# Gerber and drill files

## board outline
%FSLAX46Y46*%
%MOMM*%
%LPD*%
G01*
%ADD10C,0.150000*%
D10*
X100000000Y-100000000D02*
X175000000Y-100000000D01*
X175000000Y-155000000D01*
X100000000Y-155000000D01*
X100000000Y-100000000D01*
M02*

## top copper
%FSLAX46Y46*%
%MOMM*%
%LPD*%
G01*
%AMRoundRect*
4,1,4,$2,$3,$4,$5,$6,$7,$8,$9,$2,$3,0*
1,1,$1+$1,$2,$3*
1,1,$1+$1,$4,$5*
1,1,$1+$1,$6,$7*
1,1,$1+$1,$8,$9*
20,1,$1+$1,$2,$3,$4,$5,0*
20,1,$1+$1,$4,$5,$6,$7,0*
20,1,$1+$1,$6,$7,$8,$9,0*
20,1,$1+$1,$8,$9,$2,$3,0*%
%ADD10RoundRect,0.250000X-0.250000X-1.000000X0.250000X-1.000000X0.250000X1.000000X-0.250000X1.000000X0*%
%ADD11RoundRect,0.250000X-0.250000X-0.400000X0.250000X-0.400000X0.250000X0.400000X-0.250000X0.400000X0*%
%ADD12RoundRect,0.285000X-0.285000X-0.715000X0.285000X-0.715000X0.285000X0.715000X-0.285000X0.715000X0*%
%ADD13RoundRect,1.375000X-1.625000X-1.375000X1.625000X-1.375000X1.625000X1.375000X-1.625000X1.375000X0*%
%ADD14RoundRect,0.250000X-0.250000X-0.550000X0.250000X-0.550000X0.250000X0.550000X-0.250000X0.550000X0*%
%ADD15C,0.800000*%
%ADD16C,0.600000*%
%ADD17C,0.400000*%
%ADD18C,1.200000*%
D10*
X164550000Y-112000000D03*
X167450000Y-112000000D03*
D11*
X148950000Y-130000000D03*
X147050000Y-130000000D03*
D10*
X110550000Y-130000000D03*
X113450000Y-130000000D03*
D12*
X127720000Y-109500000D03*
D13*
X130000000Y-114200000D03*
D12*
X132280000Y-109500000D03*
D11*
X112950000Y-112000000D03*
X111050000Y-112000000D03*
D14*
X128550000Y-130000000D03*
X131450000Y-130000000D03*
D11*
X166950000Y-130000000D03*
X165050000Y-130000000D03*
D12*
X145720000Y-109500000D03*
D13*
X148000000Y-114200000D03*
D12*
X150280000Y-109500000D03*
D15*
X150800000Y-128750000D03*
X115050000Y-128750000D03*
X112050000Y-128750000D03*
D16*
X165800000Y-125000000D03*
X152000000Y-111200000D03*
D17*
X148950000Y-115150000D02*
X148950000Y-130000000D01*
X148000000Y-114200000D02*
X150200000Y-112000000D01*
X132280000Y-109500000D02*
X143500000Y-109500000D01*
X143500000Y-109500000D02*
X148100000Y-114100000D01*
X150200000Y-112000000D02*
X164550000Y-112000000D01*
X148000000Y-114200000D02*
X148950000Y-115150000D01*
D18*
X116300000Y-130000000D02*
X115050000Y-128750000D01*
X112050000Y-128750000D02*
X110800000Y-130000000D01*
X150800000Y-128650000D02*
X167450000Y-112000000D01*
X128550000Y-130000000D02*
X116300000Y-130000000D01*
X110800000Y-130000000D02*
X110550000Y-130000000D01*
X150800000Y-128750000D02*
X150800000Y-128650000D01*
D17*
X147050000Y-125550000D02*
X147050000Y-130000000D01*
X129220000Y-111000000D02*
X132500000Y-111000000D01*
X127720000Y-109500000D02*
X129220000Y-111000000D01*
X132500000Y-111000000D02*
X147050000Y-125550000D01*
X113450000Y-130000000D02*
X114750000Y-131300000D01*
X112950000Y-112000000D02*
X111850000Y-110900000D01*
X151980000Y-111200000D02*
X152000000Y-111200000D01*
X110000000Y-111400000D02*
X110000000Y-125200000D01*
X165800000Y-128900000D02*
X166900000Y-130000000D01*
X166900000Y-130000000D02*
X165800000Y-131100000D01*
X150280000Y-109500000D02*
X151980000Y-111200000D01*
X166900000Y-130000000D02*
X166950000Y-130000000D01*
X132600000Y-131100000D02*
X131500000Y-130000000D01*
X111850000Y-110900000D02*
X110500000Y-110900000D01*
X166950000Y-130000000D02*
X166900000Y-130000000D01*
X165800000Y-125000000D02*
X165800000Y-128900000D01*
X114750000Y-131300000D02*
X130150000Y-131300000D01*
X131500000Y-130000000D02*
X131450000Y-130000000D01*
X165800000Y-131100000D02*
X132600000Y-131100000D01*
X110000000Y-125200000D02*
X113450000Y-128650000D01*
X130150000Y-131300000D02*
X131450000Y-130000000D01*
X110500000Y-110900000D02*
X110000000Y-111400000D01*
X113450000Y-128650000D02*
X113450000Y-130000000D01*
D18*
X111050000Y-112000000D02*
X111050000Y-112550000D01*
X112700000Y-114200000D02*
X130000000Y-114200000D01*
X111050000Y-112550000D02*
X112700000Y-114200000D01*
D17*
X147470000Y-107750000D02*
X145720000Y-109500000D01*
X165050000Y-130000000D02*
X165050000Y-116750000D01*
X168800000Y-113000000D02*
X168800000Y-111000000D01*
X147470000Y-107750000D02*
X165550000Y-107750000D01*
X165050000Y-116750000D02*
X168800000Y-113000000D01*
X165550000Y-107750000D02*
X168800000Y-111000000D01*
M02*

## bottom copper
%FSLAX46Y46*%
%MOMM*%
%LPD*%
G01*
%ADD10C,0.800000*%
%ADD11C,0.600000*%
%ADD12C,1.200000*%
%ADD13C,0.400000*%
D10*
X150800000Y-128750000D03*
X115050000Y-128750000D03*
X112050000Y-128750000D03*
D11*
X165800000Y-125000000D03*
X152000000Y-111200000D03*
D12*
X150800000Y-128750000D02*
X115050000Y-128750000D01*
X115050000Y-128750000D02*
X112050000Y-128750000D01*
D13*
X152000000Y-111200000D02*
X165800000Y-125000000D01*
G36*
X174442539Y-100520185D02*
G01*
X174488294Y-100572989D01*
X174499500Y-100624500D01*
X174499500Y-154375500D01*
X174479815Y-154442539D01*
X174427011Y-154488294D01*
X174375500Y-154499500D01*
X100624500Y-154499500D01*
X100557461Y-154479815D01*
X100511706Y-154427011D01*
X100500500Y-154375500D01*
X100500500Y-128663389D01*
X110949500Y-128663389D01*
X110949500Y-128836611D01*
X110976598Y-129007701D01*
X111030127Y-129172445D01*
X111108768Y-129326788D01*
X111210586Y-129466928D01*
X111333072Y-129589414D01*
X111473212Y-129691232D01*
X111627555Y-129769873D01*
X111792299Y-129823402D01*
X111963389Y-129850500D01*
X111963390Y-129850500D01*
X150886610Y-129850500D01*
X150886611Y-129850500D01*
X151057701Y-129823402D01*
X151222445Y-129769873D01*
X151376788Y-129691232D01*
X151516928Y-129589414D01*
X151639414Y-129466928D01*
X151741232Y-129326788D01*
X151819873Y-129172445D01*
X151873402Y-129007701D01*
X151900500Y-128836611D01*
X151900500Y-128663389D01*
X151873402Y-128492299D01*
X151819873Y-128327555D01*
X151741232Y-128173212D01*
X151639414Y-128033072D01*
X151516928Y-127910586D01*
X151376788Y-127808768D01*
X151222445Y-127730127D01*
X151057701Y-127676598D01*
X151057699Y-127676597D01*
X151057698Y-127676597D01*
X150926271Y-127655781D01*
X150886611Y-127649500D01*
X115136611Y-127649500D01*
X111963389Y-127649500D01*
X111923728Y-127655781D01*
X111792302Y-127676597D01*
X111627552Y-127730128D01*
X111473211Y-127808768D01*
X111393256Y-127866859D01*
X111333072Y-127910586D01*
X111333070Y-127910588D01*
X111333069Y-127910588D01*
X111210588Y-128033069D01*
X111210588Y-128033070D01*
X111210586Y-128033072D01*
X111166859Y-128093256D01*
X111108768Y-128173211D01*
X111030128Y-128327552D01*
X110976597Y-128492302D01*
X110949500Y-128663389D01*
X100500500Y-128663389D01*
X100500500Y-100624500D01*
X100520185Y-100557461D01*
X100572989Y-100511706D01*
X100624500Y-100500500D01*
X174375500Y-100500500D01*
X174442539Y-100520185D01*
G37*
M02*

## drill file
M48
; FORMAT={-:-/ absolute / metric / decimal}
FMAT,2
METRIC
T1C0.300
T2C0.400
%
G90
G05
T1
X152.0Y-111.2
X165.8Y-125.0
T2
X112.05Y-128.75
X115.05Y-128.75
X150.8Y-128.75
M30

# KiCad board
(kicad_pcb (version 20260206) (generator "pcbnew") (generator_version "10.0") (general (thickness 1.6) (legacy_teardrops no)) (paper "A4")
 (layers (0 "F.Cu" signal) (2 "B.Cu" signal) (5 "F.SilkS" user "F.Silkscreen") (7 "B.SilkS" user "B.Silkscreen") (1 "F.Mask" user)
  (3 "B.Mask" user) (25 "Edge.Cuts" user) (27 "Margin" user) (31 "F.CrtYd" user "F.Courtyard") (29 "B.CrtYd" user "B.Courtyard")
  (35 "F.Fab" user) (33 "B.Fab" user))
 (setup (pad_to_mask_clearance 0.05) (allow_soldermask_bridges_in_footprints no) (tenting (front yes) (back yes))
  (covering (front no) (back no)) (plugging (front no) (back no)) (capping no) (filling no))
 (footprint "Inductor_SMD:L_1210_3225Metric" (layer "F.Cu") (at 166 112)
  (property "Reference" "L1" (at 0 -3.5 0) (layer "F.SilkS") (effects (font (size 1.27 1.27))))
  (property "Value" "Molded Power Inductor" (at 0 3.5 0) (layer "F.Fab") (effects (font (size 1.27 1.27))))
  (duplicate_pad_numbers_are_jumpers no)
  (pad "1" smd roundrect (at -1.45 0) (size 1 2.5) (layers "F.Cu" "F.Mask" "F.Paste") (roundrect_rratio 0.25) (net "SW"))
  (pad "2" smd roundrect (at 1.45 0) (size 1 2.5) (layers "F.Cu" "F.Mask" "F.Paste") (roundrect_rratio 0.25) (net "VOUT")))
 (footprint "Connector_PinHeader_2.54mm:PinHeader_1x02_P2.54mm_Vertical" (layer "F.Cu") (at 148 130)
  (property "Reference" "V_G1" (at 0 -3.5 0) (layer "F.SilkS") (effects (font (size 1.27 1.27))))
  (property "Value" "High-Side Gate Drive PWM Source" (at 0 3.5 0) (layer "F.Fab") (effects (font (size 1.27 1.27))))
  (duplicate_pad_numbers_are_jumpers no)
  (pad "n" smd roundrect (at 0.95 0) (size 1 1.3) (layers "F.Cu" "F.Mask" "F.Paste") (roundrect_rratio 0.25) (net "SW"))
  (pad "p" smd roundrect (at -0.95 0) (size 1 1.3) (layers "F.Cu" "F.Mask" "F.Paste") (roundrect_rratio 0.25) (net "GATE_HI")))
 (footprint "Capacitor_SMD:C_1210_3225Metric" (layer "F.Cu") (at 112 130)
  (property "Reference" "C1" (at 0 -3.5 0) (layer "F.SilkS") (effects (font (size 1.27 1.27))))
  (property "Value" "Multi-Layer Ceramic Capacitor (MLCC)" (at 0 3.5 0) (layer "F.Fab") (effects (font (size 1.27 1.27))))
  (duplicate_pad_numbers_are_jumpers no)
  (pad "1" smd roundrect (at -1.45 0) (size 1 2.5) (layers "F.Cu" "F.Mask" "F.Paste") (roundrect_rratio 0.25) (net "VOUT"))
  (pad "2" smd roundrect (at 1.45 0) (size 1 2.5) (layers "F.Cu" "F.Mask" "F.Paste") (roundrect_rratio 0.25) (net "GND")))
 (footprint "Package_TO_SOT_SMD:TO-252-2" (layer "F.Cu") (at 130 112)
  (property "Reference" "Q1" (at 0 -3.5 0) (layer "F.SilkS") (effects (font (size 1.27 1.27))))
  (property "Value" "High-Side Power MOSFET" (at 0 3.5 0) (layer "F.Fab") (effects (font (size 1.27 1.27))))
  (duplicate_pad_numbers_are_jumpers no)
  (pad "1" smd roundrect (at -2.28 -2.5) (size 1.14 2) (layers "F.Cu" "F.Mask" "F.Paste") (roundrect_rratio 0.25) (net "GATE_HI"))
  (pad "2" smd roundrect (at 0 2.2) (size 6 5.5) (layers "F.Cu" "F.Mask" "F.Paste") (roundrect_rratio 0.25) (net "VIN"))
  (pad "3" smd roundrect (at 2.28 -2.5) (size 1.14 2) (layers "F.Cu" "F.Mask" "F.Paste") (roundrect_rratio 0.25) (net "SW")))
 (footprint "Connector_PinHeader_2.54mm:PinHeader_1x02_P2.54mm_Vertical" (layer "F.Cu") (at 112 112)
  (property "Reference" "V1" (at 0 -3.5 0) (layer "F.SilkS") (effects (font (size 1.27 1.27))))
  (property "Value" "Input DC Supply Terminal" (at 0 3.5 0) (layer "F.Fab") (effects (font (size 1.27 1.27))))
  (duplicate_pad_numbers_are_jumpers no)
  (pad "n" smd roundrect (at 0.95 0) (size 1 1.3) (layers "F.Cu" "F.Mask" "F.Paste") (roundrect_rratio 0.25) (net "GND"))
  (pad "p" smd roundrect (at -0.95 0) (size 1 1.3) (layers "F.Cu" "F.Mask" "F.Paste") (roundrect_rratio 0.25) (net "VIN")))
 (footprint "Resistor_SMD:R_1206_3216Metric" (layer "F.Cu") (at 130 130)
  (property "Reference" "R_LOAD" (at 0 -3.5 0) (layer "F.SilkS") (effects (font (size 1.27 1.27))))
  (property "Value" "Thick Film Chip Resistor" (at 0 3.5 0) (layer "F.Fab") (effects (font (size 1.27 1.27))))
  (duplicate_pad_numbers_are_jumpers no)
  (pad "1" smd roundrect (at -1.45 0) (size 1 1.6) (layers "F.Cu" "F.Mask" "F.Paste") (roundrect_rratio 0.25) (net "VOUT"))
  (pad "2" smd roundrect (at 1.45 0) (size 1 1.6) (layers "F.Cu" "F.Mask" "F.Paste") (roundrect_rratio 0.25) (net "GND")))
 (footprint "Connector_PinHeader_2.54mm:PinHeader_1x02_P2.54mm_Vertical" (layer "F.Cu") (at 166 130)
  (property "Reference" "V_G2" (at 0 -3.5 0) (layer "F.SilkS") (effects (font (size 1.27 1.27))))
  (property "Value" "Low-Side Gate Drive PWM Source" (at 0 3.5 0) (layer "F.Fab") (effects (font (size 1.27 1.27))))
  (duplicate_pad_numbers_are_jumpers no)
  (pad "n" smd roundrect (at 0.95 0) (size 1 1.3) (layers "F.Cu" "F.Mask" "F.Paste") (roundrect_rratio 0.25) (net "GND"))
  (pad "p" smd roundrect (at -0.95 0) (size 1 1.3) (layers "F.Cu" "F.Mask" "F.Paste") (roundrect_rratio 0.25) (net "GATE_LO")))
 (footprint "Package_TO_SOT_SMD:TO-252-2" (layer "F.Cu") (at 148 112)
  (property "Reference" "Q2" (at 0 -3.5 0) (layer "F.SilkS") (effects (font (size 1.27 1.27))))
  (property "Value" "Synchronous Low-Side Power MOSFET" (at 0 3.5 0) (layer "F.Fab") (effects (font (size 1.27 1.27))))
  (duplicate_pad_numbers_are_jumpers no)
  (pad "1" smd roundrect (at -2.28 -2.5) (size 1.14 2) (layers "F.Cu" "F.Mask" "F.Paste") (roundrect_rratio 0.25) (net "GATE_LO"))
  (pad "2" smd roundrect (at 0 2.2) (size 6 5.5) (layers "F.Cu" "F.Mask" "F.Paste") (roundrect_rratio 0.25) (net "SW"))
  (pad "3" smd roundrect (at 2.28 -2.5) (size 1.14 2) (layers "F.Cu" "F.Mask" "F.Paste") (roundrect_rratio 0.25) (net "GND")))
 (gr_rect (start 100 100) (end 175 155) (stroke (width 0.15) (type solid)) (fill no) (layer "Edge.Cuts"))
 (segment (start 148.95 115.15) (end 148.95 130) (width 0.4) (layer "F.Cu") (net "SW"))
 (segment (start 148 114.2) (end 150.2 112) (width 0.4) (layer "F.Cu") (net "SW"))
 (segment (start 132.28 109.5) (end 143.5 109.5) (width 0.4) (layer "F.Cu") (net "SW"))
 (segment (start 143.5 109.5) (end 148.1 114.1) (width 0.4) (layer "F.Cu") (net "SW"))
 (segment (start 150.2 112) (end 164.55 112) (width 0.4) (layer "F.Cu") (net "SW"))
 (segment (start 148 114.2) (end 148.95 115.15) (width 0.4) (layer "F.Cu") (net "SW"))
 (segment (start 116.3 130) (end 115.05 128.75) (width 1.2) (layer "F.Cu") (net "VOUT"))
 (segment (start 112.05 128.75) (end 110.8 130) (width 1.2) (layer "F.Cu") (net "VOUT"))
 (segment (start 150.8 128.65) (end 167.45 112) (width 1.2) (layer "F.Cu") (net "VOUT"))
 (segment (start 128.55 130) (end 116.3 130) (width 1.2) (layer "F.Cu") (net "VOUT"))
 (segment (start 110.8 130) (end 110.55 130) (width 1.2) (layer "F.Cu") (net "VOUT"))
 (segment (start 150.8 128.75) (end 150.8 128.65) (width 1.2) (layer "F.Cu") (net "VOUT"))
 (via (at 150.8 128.75) (size 0.8) (drill 0.4) (layers "F.Cu" "B.Cu") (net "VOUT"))
 (via (at 115.05 128.75) (size 0.8) (drill 0.4) (layers "F.Cu" "B.Cu") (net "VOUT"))
 (via (at 112.05 128.75) (size 0.8) (drill 0.4) (layers "F.Cu" "B.Cu") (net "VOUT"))
 (segment (start 150.8 128.75) (end 115.05 128.75) (width 1.2) (layer "B.Cu") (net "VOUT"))
 (segment (start 115.05 128.75) (end 112.05 128.75) (width 1.2) (layer "B.Cu") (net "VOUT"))
 (segment (start 147.05 125.55) (end 147.05 130) (width 0.4) (layer "F.Cu") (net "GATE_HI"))
 (segment (start 129.22 111) (end 132.5 111) (width 0.4) (layer "F.Cu") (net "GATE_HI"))
 (segment (start 127.72 109.5) (end 129.22 111) (width 0.4) (layer "F.Cu") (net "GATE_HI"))
 (segment (start 132.5 111) (end 147.05 125.55) (width 0.4) (layer "F.Cu") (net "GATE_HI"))
 (segment (start 113.45 130) (end 114.75 131.3) (width 0.4) (layer "F.Cu") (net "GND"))
 (segment (start 112.95 112) (end 111.85 110.9) (width 0.4) (layer "F.Cu") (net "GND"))
 (segment (start 151.98 111.2) (end 152 111.2) (width 0.4) (layer "F.Cu") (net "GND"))
 (segment (start 110 111.4) (end 110 125.2) (width 0.4) (layer "F.Cu") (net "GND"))
 (segment (start 165.8 128.9) (end 166.9 130) (width 0.4) (layer "F.Cu") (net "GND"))
 (segment (start 166.9 130) (end 165.8 131.1) (width 0.4) (layer "F.Cu") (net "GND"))
 (segment (start 150.28 109.5) (end 151.98 111.2) (width 0.4) (layer "F.Cu") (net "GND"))
 (segment (start 166.9 130) (end 166.95 130) (width 0.4) (layer "F.Cu") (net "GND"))
 (segment (start 132.6 131.1) (end 131.5 130) (width 0.4) (layer "F.Cu") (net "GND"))
 (segment (start 111.85 110.9) (end 110.5 110.9) (width 0.4) (layer "F.Cu") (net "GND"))
 (segment (start 166.95 130) (end 166.9 130) (width 0.4) (layer "F.Cu") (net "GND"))
 (segment (start 165.8 125) (end 165.8 128.9) (width 0.4) (layer "F.Cu") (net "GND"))
 (segment (start 114.75 131.3) (end 130.15 131.3) (width 0.4) (layer "F.Cu") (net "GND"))
 (segment (start 131.5 130) (end 131.45 130) (width 0.4) (layer "F.Cu") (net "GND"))
 (segment (start 165.8 131.1) (end 132.6 131.1) (width 0.4) (layer "F.Cu") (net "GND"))
 (segment (start 110 125.2) (end 113.45 128.65) (width 0.4) (layer "F.Cu") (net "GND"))
 (segment (start 130.15 131.3) (end 131.45 130) (width 0.4) (layer "F.Cu") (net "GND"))
 (segment (start 110.5 110.9) (end 110 111.4) (width 0.4) (layer "F.Cu") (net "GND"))
 (segment (start 113.45 128.65) (end 113.45 130) (width 0.4) (layer "F.Cu") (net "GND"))
 (via (at 165.8 125) (size 0.6) (drill 0.3) (layers "F.Cu" "B.Cu") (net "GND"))
 (via (at 152 111.2) (size 0.6) (drill 0.3) (layers "F.Cu" "B.Cu") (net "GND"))
 (segment (start 152 111.2) (end 165.8 125) (width 0.4) (layer "B.Cu") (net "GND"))
 (segment (start 111.05 112) (end 111.05 112.55) (width 1.2) (layer "F.Cu") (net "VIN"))
 (segment (start 112.7 114.2) (end 130 114.2) (width 1.2) (layer "F.Cu") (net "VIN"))
 (segment (start 111.05 112.55) (end 112.7 114.2) (width 1.2) (layer "F.Cu") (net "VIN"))
 (segment (start 147.47 107.75) (end 145.72 109.5) (width 0.4) (layer "F.Cu") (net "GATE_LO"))
 (segment (start 165.05 130) (end 165.05 116.75) (width 0.4) (layer "F.Cu") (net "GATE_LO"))
 (segment (start 168.8 113) (end 168.8 111) (width 0.4) (layer "F.Cu") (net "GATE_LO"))
 (segment (start 147.47 107.75) (end 165.55 107.75) (width 0.4) (layer "F.Cu") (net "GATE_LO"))
 (segment (start 165.05 116.75) (end 168.8 113) (width 0.4) (layer "F.Cu") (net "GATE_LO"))
 (segment (start 165.55 107.75) (end 168.8 111) (width 0.4) (layer "F.Cu") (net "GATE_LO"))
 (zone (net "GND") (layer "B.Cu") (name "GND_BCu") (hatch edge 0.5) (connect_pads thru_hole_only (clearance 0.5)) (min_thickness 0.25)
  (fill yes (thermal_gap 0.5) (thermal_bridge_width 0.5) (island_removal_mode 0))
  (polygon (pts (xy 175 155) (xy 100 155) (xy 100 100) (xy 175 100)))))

